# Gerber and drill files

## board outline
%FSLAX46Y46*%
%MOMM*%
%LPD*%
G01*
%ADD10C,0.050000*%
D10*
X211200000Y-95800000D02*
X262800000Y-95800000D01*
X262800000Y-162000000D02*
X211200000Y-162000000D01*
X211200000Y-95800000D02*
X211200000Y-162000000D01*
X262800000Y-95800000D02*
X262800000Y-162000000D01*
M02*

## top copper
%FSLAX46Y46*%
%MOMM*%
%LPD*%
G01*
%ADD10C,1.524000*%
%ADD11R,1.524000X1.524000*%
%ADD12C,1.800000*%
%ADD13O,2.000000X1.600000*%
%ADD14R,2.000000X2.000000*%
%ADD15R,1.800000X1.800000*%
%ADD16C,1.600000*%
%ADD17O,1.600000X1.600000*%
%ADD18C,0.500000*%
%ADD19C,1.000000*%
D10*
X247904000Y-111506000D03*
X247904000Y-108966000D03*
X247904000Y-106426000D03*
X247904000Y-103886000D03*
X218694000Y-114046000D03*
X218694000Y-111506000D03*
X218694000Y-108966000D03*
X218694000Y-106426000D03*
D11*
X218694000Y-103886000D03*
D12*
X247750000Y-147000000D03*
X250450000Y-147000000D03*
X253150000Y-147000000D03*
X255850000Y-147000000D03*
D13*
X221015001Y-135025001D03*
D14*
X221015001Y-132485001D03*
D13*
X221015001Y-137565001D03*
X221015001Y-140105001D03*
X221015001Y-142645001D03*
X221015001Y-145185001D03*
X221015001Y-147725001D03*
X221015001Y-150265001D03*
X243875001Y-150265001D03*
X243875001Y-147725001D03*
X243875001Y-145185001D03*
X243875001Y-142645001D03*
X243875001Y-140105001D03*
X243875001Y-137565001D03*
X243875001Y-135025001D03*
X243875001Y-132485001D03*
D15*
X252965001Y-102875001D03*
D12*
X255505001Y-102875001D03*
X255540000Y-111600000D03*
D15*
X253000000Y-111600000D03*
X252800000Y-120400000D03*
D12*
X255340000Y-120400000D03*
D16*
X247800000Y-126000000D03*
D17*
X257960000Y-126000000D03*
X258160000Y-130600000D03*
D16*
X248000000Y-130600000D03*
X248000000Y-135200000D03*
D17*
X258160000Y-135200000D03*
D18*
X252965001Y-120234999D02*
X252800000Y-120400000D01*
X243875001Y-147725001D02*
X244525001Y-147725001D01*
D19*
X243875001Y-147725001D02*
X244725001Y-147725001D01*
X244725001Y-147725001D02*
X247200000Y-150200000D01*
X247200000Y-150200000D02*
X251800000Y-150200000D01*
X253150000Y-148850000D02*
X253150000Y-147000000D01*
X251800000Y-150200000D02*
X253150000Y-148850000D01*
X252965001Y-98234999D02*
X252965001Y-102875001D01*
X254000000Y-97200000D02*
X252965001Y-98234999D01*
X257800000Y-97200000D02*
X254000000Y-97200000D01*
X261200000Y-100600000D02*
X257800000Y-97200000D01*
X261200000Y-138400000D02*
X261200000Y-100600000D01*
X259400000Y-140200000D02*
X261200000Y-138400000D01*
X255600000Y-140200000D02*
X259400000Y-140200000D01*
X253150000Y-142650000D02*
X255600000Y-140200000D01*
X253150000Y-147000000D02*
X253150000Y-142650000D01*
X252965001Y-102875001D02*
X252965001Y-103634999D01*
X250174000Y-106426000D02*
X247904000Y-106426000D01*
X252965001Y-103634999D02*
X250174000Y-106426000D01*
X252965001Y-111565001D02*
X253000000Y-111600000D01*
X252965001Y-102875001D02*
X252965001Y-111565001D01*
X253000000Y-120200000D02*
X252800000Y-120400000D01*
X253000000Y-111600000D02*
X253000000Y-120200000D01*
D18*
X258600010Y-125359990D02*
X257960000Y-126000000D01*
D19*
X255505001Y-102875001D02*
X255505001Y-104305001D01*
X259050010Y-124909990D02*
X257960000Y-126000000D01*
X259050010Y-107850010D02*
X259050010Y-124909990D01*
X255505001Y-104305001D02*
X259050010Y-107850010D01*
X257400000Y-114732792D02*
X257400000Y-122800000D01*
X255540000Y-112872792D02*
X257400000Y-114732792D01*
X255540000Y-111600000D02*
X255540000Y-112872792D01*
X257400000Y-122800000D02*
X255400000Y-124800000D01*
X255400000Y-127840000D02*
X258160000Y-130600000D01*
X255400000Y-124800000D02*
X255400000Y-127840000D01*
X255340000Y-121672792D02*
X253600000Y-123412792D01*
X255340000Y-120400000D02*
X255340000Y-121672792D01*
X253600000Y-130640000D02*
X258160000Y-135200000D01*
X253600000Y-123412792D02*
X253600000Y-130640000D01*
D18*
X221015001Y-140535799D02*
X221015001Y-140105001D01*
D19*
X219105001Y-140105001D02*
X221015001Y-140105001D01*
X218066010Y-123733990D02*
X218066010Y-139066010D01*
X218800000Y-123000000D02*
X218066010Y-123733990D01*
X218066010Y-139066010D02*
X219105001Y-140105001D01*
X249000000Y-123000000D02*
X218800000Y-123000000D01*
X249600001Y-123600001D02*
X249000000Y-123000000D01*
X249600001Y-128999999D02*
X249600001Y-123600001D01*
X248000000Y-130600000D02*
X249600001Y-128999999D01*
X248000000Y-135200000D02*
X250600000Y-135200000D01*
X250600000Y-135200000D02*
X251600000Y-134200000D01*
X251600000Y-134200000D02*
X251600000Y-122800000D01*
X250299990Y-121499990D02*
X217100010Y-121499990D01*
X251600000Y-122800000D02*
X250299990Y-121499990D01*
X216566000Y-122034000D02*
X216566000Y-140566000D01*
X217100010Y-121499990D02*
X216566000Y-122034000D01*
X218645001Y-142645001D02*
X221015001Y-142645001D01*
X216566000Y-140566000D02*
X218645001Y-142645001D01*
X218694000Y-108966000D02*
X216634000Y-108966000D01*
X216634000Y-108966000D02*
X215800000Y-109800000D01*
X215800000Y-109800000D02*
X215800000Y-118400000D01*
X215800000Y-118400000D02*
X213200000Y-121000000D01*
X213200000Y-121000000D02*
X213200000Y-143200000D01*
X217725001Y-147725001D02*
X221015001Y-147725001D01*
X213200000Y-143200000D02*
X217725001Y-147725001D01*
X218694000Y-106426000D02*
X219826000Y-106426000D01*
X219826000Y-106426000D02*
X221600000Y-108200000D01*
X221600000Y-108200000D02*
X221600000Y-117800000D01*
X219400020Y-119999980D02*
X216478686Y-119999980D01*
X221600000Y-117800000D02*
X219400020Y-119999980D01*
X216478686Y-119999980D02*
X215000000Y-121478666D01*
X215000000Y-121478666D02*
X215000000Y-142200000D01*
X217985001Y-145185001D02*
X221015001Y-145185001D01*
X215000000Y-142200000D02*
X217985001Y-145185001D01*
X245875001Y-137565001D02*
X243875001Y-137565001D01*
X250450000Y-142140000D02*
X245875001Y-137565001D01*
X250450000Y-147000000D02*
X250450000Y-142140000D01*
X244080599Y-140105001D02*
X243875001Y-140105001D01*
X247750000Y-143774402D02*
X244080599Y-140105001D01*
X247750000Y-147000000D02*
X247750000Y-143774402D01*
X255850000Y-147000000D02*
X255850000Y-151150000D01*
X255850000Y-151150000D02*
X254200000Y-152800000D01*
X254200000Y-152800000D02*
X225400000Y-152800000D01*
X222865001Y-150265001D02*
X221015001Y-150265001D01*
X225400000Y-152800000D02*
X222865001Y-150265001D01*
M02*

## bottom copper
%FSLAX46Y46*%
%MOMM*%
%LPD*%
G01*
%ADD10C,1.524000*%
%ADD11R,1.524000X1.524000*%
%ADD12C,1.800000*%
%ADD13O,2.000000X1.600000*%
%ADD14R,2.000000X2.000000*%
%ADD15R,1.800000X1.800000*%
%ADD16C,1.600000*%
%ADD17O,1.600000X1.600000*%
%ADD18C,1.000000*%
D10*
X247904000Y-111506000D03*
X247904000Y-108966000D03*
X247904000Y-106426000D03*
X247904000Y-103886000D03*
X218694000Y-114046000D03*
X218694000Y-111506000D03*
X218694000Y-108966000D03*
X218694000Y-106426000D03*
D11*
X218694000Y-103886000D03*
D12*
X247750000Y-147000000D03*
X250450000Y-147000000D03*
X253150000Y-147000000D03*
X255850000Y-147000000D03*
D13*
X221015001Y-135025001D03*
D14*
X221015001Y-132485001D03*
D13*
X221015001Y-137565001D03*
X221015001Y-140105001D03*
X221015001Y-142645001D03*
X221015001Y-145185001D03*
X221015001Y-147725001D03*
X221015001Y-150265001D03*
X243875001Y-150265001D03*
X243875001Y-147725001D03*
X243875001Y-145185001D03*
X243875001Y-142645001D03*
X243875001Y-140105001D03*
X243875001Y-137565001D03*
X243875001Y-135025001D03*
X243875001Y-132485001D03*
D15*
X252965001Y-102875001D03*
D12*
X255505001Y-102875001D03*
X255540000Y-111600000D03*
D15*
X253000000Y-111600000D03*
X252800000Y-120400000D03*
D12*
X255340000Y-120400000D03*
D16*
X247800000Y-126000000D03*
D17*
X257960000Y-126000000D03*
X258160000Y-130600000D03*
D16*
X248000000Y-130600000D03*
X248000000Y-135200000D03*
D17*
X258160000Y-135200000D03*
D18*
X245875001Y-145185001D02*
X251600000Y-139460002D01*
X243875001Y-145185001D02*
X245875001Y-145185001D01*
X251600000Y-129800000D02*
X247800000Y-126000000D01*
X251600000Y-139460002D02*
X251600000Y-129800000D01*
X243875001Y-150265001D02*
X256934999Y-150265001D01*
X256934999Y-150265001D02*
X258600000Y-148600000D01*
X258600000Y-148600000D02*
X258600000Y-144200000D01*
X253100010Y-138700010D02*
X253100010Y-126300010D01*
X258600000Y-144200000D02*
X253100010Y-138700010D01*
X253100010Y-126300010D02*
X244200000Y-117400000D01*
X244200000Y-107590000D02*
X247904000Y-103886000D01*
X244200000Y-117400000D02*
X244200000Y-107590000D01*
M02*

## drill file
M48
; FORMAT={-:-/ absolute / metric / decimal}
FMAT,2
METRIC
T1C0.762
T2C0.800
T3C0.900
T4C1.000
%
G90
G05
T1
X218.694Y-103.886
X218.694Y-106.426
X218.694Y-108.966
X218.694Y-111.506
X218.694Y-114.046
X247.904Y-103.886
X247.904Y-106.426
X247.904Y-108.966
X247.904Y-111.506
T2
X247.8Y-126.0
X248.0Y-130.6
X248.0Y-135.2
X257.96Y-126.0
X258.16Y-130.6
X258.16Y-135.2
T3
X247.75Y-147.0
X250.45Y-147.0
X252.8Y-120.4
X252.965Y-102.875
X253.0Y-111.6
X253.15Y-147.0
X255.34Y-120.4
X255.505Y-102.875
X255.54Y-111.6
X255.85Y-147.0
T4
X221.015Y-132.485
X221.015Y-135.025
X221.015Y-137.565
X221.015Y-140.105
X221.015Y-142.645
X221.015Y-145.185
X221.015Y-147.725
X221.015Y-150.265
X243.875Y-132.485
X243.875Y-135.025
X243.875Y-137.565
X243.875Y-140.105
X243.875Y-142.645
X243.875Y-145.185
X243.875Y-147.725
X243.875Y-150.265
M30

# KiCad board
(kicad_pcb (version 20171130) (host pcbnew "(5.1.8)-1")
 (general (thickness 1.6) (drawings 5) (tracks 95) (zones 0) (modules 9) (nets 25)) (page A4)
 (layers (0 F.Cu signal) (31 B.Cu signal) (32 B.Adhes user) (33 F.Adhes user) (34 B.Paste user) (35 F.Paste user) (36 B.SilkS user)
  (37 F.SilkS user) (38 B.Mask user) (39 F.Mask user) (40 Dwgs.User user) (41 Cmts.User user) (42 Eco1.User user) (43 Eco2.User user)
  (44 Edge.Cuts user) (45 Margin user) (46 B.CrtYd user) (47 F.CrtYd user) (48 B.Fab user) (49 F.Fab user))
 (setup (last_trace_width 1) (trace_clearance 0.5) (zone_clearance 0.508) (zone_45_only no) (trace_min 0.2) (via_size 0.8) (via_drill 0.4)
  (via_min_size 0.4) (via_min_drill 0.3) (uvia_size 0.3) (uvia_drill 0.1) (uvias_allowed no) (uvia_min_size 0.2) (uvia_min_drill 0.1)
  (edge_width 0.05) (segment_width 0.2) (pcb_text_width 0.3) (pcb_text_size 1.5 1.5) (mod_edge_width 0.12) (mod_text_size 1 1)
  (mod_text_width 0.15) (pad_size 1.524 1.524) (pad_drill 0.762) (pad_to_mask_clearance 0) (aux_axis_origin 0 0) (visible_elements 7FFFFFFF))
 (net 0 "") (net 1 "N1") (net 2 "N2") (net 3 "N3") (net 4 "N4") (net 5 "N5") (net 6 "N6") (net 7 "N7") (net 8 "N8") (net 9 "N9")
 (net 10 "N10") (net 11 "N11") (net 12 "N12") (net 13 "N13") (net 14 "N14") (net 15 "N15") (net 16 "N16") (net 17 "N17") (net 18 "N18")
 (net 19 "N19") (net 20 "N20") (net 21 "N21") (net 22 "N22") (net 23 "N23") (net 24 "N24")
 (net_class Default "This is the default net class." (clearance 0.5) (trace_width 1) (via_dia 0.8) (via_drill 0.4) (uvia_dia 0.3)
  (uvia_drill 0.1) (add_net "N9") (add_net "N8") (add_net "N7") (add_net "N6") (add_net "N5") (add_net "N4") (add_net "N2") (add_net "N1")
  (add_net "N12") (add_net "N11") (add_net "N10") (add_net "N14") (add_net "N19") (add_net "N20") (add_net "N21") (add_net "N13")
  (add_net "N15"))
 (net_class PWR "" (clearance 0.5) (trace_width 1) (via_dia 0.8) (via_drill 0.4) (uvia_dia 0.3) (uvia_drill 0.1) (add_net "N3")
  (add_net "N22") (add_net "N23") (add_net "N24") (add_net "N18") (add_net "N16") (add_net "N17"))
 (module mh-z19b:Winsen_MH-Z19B (layer F.Cu) (at 218.694 117.856 180)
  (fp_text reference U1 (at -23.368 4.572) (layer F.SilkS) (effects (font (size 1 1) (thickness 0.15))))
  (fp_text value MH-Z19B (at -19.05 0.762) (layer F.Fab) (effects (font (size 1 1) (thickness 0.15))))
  (pad 9 thru_hole circle (at -29.21 6.35 180) (size 1.524 1.524) (drill 0.762) (layers *.Cu *.Mask) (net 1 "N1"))
  (pad 8 thru_hole circle (at -29.21 8.89 180) (size 1.524 1.524) (drill 0.762) (layers *.Cu *.Mask) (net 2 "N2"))
  (pad 7 thru_hole circle (at -29.21 11.43 180) (size 1.524 1.524) (drill 0.762) (layers *.Cu *.Mask) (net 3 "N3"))
  (pad 6 thru_hole circle (at -29.21 13.97 180) (size 1.524 1.524) (drill 0.762) (layers *.Cu *.Mask) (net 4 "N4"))
  (pad 5 thru_hole circle (at 0 3.81 180) (size 1.524 1.524) (drill 0.762) (layers *.Cu *.Mask) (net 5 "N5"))
  (pad 4 thru_hole circle (at 0 6.35 180) (size 1.524 1.524) (drill 0.762) (layers *.Cu *.Mask) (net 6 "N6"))
  (pad 3 thru_hole circle (at 0 8.89 180) (size 1.524 1.524) (drill 0.762) (layers *.Cu *.Mask) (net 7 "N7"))
  (pad 2 thru_hole circle (at 0 11.43 180) (size 1.524 1.524) (drill 0.762) (layers *.Cu *.Mask) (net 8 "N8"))
  (pad 1 thru_hole rect (at 0 13.97 180) (size 1.524 1.524) (drill 0.762) (layers *.Cu *.Mask) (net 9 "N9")))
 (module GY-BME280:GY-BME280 (layer F.Cu) (at 251.8 149 180)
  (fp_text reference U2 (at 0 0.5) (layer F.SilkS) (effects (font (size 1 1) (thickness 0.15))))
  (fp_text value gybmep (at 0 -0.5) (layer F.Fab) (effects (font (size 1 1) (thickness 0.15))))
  (pad 4 thru_hole circle (at 4.05 2 180) (size 1.8 1.8) (drill 0.9) (layers *.Cu *.Mask) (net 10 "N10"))
  (pad 3 thru_hole circle (at 1.35 2 180) (size 1.8 1.8) (drill 0.9) (layers *.Cu *.Mask) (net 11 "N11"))
  (pad 2 thru_hole circle (at -1.35 2 180) (size 1.8 1.8) (drill 0.9) (layers *.Cu *.Mask) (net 3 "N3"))
  (pad 1 thru_hole circle (at -4.05 2 180) (size 1.8 1.8) (drill 0.9) (layers *.Cu *.Mask) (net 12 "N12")))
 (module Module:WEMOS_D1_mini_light (layer F.Cu) (at 221.015001 132.485001)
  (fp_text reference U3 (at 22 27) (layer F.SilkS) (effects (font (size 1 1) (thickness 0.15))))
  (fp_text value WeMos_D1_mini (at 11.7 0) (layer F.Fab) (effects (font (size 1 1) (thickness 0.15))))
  (pad 2 thru_hole oval (at 0 2.54) (size 2 1.6) (drill 1) (layers *.Cu *.Mask) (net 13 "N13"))
  (pad 1 thru_hole rect (at 0 0) (size 2 2) (drill 1) (layers *.Cu *.Mask) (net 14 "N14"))
  (pad 3 thru_hole oval (at 0 5.08) (size 2 1.6) (drill 1) (layers *.Cu *.Mask) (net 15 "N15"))
  (pad 4 thru_hole oval (at 0 7.62) (size 2 1.6) (drill 1) (layers *.Cu *.Mask) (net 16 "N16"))
  (pad 5 thru_hole oval (at 0 10.16) (size 2 1.6) (drill 1) (layers *.Cu *.Mask) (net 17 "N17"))
  (pad 6 thru_hole oval (at 0 12.7) (size 2 1.6) (drill 1) (layers *.Cu *.Mask) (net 8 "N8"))
  (pad 7 thru_hole oval (at 0 15.24) (size 2 1.6) (drill 1) (layers *.Cu *.Mask) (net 7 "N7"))
  (pad 8 thru_hole oval (at 0 17.78) (size 2 1.6) (drill 1) (layers *.Cu *.Mask) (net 12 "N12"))
  (pad 9 thru_hole oval (at 22.86 17.78) (size 2 1.6) (drill 1) (layers *.Cu *.Mask) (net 4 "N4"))
  (pad 10 thru_hole oval (at 22.86 15.24) (size 2 1.6) (drill 1) (layers *.Cu *.Mask) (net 3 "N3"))
  (pad 11 thru_hole oval (at 22.86 12.7) (size 2 1.6) (drill 1) (layers *.Cu *.Mask) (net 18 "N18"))
  (pad 12 thru_hole oval (at 22.86 10.16) (size 2 1.6) (drill 1) (layers *.Cu *.Mask) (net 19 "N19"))
  (pad 13 thru_hole oval (at 22.86 7.62) (size 2 1.6) (drill 1) (layers *.Cu *.Mask) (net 10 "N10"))
  (pad 14 thru_hole oval (at 22.86 5.08) (size 2 1.6) (drill 1) (layers *.Cu *.Mask) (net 11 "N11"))
  (pad 15 thru_hole oval (at 22.86 2.54) (size 2 1.6) (drill 1) (layers *.Cu *.Mask) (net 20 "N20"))
  (pad 16 thru_hole oval (at 22.86 0) (size 2 1.6) (drill 1) (layers *.Cu *.Mask) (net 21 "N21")))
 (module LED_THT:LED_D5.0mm (layer F.Cu) (at 252.965001 102.875001)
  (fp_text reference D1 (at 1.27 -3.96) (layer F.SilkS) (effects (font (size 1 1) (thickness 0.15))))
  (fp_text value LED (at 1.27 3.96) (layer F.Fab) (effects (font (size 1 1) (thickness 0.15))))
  (pad 1 thru_hole rect (at 0 0) (size 1.8 1.8) (drill 0.9) (layers *.Cu *.Mask) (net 3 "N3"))
  (pad 2 thru_hole circle (at 2.54 0) (size 1.8 1.8) (drill 0.9) (layers *.Cu *.Mask) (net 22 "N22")))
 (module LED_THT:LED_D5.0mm (layer F.Cu) (at 253 111.6)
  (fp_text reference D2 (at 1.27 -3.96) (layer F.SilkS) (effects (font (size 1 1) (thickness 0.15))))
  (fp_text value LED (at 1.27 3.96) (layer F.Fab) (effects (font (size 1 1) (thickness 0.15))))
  (pad 2 thru_hole circle (at 2.54 0) (size 1.8 1.8) (drill 0.9) (layers *.Cu *.Mask) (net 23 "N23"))
  (pad 1 thru_hole rect (at 0 0) (size 1.8 1.8) (drill 0.9) (layers *.Cu *.Mask) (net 3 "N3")))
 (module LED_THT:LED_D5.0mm (layer F.Cu) (at 252.8 120.4)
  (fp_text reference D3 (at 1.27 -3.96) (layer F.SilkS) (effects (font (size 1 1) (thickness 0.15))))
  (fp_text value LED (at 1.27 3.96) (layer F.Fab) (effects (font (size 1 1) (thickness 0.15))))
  (pad 1 thru_hole rect (at 0 0) (size 1.8 1.8) (drill 0.9) (layers *.Cu *.Mask) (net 3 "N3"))
  (pad 2 thru_hole circle (at 2.54 0) (size 1.8 1.8) (drill 0.9) (layers *.Cu *.Mask) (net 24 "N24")))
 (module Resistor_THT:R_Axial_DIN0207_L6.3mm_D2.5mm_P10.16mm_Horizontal (layer F.Cu) (at 247.8 126)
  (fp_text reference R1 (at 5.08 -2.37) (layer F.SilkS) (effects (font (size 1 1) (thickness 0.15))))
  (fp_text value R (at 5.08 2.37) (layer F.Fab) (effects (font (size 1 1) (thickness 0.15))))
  (pad 1 thru_hole circle (at 0 0) (size 1.6 1.6) (drill 0.8) (layers *.Cu *.Mask) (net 18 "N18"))
  (pad 2 thru_hole oval (at 10.16 0) (size 1.6 1.6) (drill 0.8) (layers *.Cu *.Mask) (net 22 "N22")))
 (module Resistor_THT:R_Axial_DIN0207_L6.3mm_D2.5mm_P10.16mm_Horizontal (layer F.Cu) (at 248 130.6)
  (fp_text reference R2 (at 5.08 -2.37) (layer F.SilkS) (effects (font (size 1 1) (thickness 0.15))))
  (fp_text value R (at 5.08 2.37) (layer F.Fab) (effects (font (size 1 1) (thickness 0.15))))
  (pad 2 thru_hole oval (at 10.16 0) (size 1.6 1.6) (drill 0.8) (layers *.Cu *.Mask) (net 23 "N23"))
  (pad 1 thru_hole circle (at 0 0) (size 1.6 1.6) (drill 0.8) (layers *.Cu *.Mask) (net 16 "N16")))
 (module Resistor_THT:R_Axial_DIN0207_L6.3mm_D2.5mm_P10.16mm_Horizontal (layer F.Cu) (at 248 135.2)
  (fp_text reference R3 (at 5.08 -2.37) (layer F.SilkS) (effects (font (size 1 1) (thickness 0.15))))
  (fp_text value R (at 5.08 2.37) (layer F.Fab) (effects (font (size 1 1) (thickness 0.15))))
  (pad 1 thru_hole circle (at 0 0) (size 1.6 1.6) (drill 0.8) (layers *.Cu *.Mask) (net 17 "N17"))
  (pad 2 thru_hole oval (at 10.16 0) (size 1.6 1.6) (drill 0.8) (layers *.Cu *.Mask) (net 24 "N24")))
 (gr_line (start 211.2 95.8) (end 262.8 95.8) (layer Edge.Cuts) (width 0.05))
 (gr_line (start 262.8 162) (end 211.2 162) (layer Edge.Cuts) (width 0.05))
 (gr_line (start 211.2 95.8) (end 211.2 162) (layer Edge.Cuts) (width 0.05))
 (gr_line (start 262.8 95.8) (end 262.8 162) (layer Edge.Cuts) (width 0.05))
 (segment (start 252.965001 120.234999) (end 252.8 120.4) (width 0.5) (layer F.Cu) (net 3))
 (segment (start 243.875001 147.725001) (end 244.525001 147.725001) (width 0.5) (layer F.Cu) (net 3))
 (segment (start 243.875001 147.725001) (end 244.725001 147.725001) (width 1) (layer F.Cu) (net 3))
 (segment (start 244.725001 147.725001) (end 247.2 150.2) (width 1) (layer F.Cu) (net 3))
 (segment (start 247.2 150.2) (end 251.8 150.2) (width 1) (layer F.Cu) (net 3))
 (segment (start 253.15 148.85) (end 253.15 147) (width 1) (layer F.Cu) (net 3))
 (segment (start 251.8 150.2) (end 253.15 148.85) (width 1) (layer F.Cu) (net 3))
 (segment (start 252.965001 98.234999) (end 252.965001 102.875001) (width 1) (layer F.Cu) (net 3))
 (segment (start 254 97.2) (end 252.965001 98.234999) (width 1) (layer F.Cu) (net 3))
 (segment (start 257.8 97.2) (end 254 97.2) (width 1) (layer F.Cu) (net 3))
 (segment (start 261.2 100.6) (end 257.8 97.2) (width 1) (layer F.Cu) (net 3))
 (segment (start 261.2 138.4) (end 261.2 100.6) (width 1) (layer F.Cu) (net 3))
 (segment (start 259.4 140.2) (end 261.2 138.4) (width 1) (layer F.Cu) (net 3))
 (segment (start 255.6 140.2) (end 259.4 140.2) (width 1) (layer F.Cu) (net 3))
 (segment (start 253.15 142.65) (end 255.6 140.2) (width 1) (layer F.Cu) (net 3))
 (segment (start 253.15 147) (end 253.15 142.65) (width 1) (layer F.Cu) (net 3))
 (segment (start 252.965001 102.875001) (end 252.965001 103.634999) (width 1) (layer F.Cu) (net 3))
 (segment (start 250.174 106.426) (end 247.904 106.426) (width 1) (layer F.Cu) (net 3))
 (segment (start 252.965001 103.634999) (end 250.174 106.426) (width 1) (layer F.Cu) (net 3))
 (segment (start 252.965001 111.565001) (end 253 111.6) (width 1) (layer F.Cu) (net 3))
 (segment (start 252.965001 102.875001) (end 252.965001 111.565001) (width 1) (layer F.Cu) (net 3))
 (segment (start 253 120.2) (end 252.8 120.4) (width 1) (layer F.Cu) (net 3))
 (segment (start 253 111.6) (end 253 120.2) (width 1) (layer F.Cu) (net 3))
 (segment (start 258.60001 125.35999) (end 257.96 126) (width 0.5) (layer F.Cu) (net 22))
 (segment (start 255.505001 102.875001) (end 255.505001 104.305001) (width 1) (layer F.Cu) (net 22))
 (segment (start 259.05001 124.90999) (end 257.96 126) (width 1) (layer F.Cu) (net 22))
 (segment (start 259.05001 107.85001) (end 259.05001 124.90999) (width 1) (layer F.Cu) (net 22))
 (segment (start 255.505001 104.305001) (end 259.05001 107.85001) (width 1) (layer F.Cu) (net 22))
 (segment (start 257.4 114.732792) (end 257.4 122.8) (width 1) (layer F.Cu) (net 23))
 (segment (start 255.54 112.872792) (end 257.4 114.732792) (width 1) (layer F.Cu) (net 23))
 (segment (start 255.54 111.6) (end 255.54 112.872792) (width 1) (layer F.Cu) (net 23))
 (segment (start 257.4 122.8) (end 255.4 124.8) (width 1) (layer F.Cu) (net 23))
 (segment (start 255.4 127.84) (end 258.16 130.6) (width 1) (layer F.Cu) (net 23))
 (segment (start 255.4 124.8) (end 255.4 127.84) (width 1) (layer F.Cu) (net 23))
 (segment (start 255.34 121.672792) (end 253.6 123.412792) (width 1) (layer F.Cu) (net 24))
 (segment (start 255.34 120.4) (end 255.34 121.672792) (width 1) (layer F.Cu) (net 24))
 (segment (start 253.6 130.64) (end 258.16 135.2) (width 1) (layer F.Cu) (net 24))
 (segment (start 253.6 123.412792) (end 253.6 130.64) (width 1) (layer F.Cu) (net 24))
 (segment (start 245.875001 145.185001) (end 251.6 139.460002) (width 1) (layer B.Cu) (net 18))
 (segment (start 243.875001 145.185001) (end 245.875001 145.185001) (width 1) (layer B.Cu) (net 18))
 (segment (start 251.6 129.8) (end 247.8 126) (width 1) (layer B.Cu) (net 18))
 (segment (start 251.6 139.460002) (end 251.6 129.8) (width 1) (layer B.Cu) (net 18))
 (segment (start 221.015001 140.535799) (end 221.015001 140.105001) (width 0.5) (layer F.Cu) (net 16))
 (segment (start 219.105001 140.105001) (end 221.015001 140.105001) (width 1) (layer F.Cu) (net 16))
 (segment (start 218.06601 123.73399) (end 218.06601 139.06601) (width 1) (layer F.Cu) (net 16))
 (segment (start 218.8 123) (end 218.06601 123.73399) (width 1) (layer F.Cu) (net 16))
 (segment (start 218.06601 139.06601) (end 219.105001 140.105001) (width 1) (layer F.Cu) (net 16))
 (segment (start 249 123) (end 218.8 123) (width 1) (layer F.Cu) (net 16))
 (segment (start 249.600001 123.600001) (end 249 123) (width 1) (layer F.Cu) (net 16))
 (segment (start 249.600001 128.999999) (end 249.600001 123.600001) (width 1) (layer F.Cu) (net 16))
 (segment (start 248 130.6) (end 249.600001 128.999999) (width 1) (layer F.Cu) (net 16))
 (segment (start 248 135.2) (end 250.6 135.2) (width 1) (layer F.Cu) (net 17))
 (segment (start 250.6 135.2) (end 251.6 134.2) (width 1) (layer F.Cu) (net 17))
 (segment (start 251.6 134.2) (end 251.6 122.8) (width 1) (layer F.Cu) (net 17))
 (segment (start 250.29999 121.49999) (end 217.10001 121.49999) (width 1) (layer F.Cu) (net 17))
 (segment (start 251.6 122.8) (end 250.29999 121.49999) (width 1) (layer F.Cu) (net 17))
 (segment (start 216.566 122.034) (end 216.566 140.566) (width 1) (layer F.Cu) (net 17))
 (segment (start 217.10001 121.49999) (end 216.566 122.034) (width 1) (layer F.Cu) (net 17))
 (segment (start 218.645001 142.645001) (end 221.015001 142.645001) (width 1) (layer F.Cu) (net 17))
 (segment (start 216.566 140.566) (end 218.645001 142.645001) (width 1) (layer F.Cu) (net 17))
 (segment (start 243.875001 150.265001) (end 256.934999 150.265001) (width 1) (layer B.Cu) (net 4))
 (segment (start 256.934999 150.265001) (end 258.6 148.6) (width 1) (layer B.Cu) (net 4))
 (segment (start 258.6 148.6) (end 258.6 144.2) (width 1) (layer B.Cu) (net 4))
 (segment (start 253.10001 138.70001) (end 253.10001 126.30001) (width 1) (layer B.Cu) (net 4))
 (segment (start 258.6 144.2) (end 253.10001 138.70001) (width 1) (layer B.Cu) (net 4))
 (segment (start 253.10001 126.30001) (end 244.2 117.4) (width 1) (layer B.Cu) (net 4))
 (segment (start 244.2 107.59) (end 247.904 103.886) (width 1) (layer B.Cu) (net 4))
 (segment (start 244.2 117.4) (end 244.2 107.59) (width 1) (layer B.Cu) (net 4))
 (segment (start 218.694 108.966) (end 216.634 108.966) (width 1) (layer F.Cu) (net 7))
 (segment (start 216.634 108.966) (end 215.8 109.8) (width 1) (layer F.Cu) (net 7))
 (segment (start 215.8 109.8) (end 215.8 118.4) (width 1) (layer F.Cu) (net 7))
 (segment (start 215.8 118.4) (end 213.2 121) (width 1) (layer F.Cu) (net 7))
 (segment (start 213.2 121) (end 213.2 143.2) (width 1) (layer F.Cu) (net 7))
 (segment (start 217.725001 147.725001) (end 221.015001 147.725001) (width 1) (layer F.Cu) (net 7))
 (segment (start 213.2 143.2) (end 217.725001 147.725001) (width 1) (layer F.Cu) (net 7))
 (segment (start 218.694 106.426) (end 219.826 106.426) (width 1) (layer F.Cu) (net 8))
 (segment (start 219.826 106.426) (end 221.6 108.2) (width 1) (layer F.Cu) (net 8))
 (segment (start 221.6 108.2) (end 221.6 117.8) (width 1) (layer F.Cu) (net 8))
 (segment (start 219.40002 119.99998) (end 216.478686 119.99998) (width 1) (layer F.Cu) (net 8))
 (segment (start 221.6 117.8) (end 219.40002 119.99998) (width 1) (layer F.Cu) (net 8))
 (segment (start 216.478686 119.99998) (end 215 121.478666) (width 1) (layer F.Cu) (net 8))
 (segment (start 215 121.478666) (end 215 142.2) (width 1) (layer F.Cu) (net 8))
 (segment (start 217.985001 145.185001) (end 221.015001 145.185001) (width 1) (layer F.Cu) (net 8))
 (segment (start 215 142.2) (end 217.985001 145.185001) (width 1) (layer F.Cu) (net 8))
 (segment (start 245.875001 137.565001) (end 243.875001 137.565001) (width 1) (layer F.Cu) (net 11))
 (segment (start 250.45 142.14) (end 245.875001 137.565001) (width 1) (layer F.Cu) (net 11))
 (segment (start 250.45 147) (end 250.45 142.14) (width 1) (layer F.Cu) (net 11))
 (segment (start 244.080599 140.105001) (end 243.875001 140.105001) (width 1) (layer F.Cu) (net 10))
 (segment (start 247.75 143.774402) (end 244.080599 140.105001) (width 1) (layer F.Cu) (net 10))
 (segment (start 247.75 147) (end 247.75 143.774402) (width 1) (layer F.Cu) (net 10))
 (segment (start 255.85 147) (end 255.85 151.15) (width 1) (layer F.Cu) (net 12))
 (segment (start 255.85 151.15) (end 254.2 152.8) (width 1) (layer F.Cu) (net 12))
 (segment (start 254.2 152.8) (end 225.4 152.8) (width 1) (layer F.Cu) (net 12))
 (segment (start 222.865001 150.265001) (end 221.015001 150.265001) (width 1) (layer F.Cu) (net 12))
 (segment (start 225.4 152.8) (end 222.865001 150.265001) (width 1) (layer F.Cu) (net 12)))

